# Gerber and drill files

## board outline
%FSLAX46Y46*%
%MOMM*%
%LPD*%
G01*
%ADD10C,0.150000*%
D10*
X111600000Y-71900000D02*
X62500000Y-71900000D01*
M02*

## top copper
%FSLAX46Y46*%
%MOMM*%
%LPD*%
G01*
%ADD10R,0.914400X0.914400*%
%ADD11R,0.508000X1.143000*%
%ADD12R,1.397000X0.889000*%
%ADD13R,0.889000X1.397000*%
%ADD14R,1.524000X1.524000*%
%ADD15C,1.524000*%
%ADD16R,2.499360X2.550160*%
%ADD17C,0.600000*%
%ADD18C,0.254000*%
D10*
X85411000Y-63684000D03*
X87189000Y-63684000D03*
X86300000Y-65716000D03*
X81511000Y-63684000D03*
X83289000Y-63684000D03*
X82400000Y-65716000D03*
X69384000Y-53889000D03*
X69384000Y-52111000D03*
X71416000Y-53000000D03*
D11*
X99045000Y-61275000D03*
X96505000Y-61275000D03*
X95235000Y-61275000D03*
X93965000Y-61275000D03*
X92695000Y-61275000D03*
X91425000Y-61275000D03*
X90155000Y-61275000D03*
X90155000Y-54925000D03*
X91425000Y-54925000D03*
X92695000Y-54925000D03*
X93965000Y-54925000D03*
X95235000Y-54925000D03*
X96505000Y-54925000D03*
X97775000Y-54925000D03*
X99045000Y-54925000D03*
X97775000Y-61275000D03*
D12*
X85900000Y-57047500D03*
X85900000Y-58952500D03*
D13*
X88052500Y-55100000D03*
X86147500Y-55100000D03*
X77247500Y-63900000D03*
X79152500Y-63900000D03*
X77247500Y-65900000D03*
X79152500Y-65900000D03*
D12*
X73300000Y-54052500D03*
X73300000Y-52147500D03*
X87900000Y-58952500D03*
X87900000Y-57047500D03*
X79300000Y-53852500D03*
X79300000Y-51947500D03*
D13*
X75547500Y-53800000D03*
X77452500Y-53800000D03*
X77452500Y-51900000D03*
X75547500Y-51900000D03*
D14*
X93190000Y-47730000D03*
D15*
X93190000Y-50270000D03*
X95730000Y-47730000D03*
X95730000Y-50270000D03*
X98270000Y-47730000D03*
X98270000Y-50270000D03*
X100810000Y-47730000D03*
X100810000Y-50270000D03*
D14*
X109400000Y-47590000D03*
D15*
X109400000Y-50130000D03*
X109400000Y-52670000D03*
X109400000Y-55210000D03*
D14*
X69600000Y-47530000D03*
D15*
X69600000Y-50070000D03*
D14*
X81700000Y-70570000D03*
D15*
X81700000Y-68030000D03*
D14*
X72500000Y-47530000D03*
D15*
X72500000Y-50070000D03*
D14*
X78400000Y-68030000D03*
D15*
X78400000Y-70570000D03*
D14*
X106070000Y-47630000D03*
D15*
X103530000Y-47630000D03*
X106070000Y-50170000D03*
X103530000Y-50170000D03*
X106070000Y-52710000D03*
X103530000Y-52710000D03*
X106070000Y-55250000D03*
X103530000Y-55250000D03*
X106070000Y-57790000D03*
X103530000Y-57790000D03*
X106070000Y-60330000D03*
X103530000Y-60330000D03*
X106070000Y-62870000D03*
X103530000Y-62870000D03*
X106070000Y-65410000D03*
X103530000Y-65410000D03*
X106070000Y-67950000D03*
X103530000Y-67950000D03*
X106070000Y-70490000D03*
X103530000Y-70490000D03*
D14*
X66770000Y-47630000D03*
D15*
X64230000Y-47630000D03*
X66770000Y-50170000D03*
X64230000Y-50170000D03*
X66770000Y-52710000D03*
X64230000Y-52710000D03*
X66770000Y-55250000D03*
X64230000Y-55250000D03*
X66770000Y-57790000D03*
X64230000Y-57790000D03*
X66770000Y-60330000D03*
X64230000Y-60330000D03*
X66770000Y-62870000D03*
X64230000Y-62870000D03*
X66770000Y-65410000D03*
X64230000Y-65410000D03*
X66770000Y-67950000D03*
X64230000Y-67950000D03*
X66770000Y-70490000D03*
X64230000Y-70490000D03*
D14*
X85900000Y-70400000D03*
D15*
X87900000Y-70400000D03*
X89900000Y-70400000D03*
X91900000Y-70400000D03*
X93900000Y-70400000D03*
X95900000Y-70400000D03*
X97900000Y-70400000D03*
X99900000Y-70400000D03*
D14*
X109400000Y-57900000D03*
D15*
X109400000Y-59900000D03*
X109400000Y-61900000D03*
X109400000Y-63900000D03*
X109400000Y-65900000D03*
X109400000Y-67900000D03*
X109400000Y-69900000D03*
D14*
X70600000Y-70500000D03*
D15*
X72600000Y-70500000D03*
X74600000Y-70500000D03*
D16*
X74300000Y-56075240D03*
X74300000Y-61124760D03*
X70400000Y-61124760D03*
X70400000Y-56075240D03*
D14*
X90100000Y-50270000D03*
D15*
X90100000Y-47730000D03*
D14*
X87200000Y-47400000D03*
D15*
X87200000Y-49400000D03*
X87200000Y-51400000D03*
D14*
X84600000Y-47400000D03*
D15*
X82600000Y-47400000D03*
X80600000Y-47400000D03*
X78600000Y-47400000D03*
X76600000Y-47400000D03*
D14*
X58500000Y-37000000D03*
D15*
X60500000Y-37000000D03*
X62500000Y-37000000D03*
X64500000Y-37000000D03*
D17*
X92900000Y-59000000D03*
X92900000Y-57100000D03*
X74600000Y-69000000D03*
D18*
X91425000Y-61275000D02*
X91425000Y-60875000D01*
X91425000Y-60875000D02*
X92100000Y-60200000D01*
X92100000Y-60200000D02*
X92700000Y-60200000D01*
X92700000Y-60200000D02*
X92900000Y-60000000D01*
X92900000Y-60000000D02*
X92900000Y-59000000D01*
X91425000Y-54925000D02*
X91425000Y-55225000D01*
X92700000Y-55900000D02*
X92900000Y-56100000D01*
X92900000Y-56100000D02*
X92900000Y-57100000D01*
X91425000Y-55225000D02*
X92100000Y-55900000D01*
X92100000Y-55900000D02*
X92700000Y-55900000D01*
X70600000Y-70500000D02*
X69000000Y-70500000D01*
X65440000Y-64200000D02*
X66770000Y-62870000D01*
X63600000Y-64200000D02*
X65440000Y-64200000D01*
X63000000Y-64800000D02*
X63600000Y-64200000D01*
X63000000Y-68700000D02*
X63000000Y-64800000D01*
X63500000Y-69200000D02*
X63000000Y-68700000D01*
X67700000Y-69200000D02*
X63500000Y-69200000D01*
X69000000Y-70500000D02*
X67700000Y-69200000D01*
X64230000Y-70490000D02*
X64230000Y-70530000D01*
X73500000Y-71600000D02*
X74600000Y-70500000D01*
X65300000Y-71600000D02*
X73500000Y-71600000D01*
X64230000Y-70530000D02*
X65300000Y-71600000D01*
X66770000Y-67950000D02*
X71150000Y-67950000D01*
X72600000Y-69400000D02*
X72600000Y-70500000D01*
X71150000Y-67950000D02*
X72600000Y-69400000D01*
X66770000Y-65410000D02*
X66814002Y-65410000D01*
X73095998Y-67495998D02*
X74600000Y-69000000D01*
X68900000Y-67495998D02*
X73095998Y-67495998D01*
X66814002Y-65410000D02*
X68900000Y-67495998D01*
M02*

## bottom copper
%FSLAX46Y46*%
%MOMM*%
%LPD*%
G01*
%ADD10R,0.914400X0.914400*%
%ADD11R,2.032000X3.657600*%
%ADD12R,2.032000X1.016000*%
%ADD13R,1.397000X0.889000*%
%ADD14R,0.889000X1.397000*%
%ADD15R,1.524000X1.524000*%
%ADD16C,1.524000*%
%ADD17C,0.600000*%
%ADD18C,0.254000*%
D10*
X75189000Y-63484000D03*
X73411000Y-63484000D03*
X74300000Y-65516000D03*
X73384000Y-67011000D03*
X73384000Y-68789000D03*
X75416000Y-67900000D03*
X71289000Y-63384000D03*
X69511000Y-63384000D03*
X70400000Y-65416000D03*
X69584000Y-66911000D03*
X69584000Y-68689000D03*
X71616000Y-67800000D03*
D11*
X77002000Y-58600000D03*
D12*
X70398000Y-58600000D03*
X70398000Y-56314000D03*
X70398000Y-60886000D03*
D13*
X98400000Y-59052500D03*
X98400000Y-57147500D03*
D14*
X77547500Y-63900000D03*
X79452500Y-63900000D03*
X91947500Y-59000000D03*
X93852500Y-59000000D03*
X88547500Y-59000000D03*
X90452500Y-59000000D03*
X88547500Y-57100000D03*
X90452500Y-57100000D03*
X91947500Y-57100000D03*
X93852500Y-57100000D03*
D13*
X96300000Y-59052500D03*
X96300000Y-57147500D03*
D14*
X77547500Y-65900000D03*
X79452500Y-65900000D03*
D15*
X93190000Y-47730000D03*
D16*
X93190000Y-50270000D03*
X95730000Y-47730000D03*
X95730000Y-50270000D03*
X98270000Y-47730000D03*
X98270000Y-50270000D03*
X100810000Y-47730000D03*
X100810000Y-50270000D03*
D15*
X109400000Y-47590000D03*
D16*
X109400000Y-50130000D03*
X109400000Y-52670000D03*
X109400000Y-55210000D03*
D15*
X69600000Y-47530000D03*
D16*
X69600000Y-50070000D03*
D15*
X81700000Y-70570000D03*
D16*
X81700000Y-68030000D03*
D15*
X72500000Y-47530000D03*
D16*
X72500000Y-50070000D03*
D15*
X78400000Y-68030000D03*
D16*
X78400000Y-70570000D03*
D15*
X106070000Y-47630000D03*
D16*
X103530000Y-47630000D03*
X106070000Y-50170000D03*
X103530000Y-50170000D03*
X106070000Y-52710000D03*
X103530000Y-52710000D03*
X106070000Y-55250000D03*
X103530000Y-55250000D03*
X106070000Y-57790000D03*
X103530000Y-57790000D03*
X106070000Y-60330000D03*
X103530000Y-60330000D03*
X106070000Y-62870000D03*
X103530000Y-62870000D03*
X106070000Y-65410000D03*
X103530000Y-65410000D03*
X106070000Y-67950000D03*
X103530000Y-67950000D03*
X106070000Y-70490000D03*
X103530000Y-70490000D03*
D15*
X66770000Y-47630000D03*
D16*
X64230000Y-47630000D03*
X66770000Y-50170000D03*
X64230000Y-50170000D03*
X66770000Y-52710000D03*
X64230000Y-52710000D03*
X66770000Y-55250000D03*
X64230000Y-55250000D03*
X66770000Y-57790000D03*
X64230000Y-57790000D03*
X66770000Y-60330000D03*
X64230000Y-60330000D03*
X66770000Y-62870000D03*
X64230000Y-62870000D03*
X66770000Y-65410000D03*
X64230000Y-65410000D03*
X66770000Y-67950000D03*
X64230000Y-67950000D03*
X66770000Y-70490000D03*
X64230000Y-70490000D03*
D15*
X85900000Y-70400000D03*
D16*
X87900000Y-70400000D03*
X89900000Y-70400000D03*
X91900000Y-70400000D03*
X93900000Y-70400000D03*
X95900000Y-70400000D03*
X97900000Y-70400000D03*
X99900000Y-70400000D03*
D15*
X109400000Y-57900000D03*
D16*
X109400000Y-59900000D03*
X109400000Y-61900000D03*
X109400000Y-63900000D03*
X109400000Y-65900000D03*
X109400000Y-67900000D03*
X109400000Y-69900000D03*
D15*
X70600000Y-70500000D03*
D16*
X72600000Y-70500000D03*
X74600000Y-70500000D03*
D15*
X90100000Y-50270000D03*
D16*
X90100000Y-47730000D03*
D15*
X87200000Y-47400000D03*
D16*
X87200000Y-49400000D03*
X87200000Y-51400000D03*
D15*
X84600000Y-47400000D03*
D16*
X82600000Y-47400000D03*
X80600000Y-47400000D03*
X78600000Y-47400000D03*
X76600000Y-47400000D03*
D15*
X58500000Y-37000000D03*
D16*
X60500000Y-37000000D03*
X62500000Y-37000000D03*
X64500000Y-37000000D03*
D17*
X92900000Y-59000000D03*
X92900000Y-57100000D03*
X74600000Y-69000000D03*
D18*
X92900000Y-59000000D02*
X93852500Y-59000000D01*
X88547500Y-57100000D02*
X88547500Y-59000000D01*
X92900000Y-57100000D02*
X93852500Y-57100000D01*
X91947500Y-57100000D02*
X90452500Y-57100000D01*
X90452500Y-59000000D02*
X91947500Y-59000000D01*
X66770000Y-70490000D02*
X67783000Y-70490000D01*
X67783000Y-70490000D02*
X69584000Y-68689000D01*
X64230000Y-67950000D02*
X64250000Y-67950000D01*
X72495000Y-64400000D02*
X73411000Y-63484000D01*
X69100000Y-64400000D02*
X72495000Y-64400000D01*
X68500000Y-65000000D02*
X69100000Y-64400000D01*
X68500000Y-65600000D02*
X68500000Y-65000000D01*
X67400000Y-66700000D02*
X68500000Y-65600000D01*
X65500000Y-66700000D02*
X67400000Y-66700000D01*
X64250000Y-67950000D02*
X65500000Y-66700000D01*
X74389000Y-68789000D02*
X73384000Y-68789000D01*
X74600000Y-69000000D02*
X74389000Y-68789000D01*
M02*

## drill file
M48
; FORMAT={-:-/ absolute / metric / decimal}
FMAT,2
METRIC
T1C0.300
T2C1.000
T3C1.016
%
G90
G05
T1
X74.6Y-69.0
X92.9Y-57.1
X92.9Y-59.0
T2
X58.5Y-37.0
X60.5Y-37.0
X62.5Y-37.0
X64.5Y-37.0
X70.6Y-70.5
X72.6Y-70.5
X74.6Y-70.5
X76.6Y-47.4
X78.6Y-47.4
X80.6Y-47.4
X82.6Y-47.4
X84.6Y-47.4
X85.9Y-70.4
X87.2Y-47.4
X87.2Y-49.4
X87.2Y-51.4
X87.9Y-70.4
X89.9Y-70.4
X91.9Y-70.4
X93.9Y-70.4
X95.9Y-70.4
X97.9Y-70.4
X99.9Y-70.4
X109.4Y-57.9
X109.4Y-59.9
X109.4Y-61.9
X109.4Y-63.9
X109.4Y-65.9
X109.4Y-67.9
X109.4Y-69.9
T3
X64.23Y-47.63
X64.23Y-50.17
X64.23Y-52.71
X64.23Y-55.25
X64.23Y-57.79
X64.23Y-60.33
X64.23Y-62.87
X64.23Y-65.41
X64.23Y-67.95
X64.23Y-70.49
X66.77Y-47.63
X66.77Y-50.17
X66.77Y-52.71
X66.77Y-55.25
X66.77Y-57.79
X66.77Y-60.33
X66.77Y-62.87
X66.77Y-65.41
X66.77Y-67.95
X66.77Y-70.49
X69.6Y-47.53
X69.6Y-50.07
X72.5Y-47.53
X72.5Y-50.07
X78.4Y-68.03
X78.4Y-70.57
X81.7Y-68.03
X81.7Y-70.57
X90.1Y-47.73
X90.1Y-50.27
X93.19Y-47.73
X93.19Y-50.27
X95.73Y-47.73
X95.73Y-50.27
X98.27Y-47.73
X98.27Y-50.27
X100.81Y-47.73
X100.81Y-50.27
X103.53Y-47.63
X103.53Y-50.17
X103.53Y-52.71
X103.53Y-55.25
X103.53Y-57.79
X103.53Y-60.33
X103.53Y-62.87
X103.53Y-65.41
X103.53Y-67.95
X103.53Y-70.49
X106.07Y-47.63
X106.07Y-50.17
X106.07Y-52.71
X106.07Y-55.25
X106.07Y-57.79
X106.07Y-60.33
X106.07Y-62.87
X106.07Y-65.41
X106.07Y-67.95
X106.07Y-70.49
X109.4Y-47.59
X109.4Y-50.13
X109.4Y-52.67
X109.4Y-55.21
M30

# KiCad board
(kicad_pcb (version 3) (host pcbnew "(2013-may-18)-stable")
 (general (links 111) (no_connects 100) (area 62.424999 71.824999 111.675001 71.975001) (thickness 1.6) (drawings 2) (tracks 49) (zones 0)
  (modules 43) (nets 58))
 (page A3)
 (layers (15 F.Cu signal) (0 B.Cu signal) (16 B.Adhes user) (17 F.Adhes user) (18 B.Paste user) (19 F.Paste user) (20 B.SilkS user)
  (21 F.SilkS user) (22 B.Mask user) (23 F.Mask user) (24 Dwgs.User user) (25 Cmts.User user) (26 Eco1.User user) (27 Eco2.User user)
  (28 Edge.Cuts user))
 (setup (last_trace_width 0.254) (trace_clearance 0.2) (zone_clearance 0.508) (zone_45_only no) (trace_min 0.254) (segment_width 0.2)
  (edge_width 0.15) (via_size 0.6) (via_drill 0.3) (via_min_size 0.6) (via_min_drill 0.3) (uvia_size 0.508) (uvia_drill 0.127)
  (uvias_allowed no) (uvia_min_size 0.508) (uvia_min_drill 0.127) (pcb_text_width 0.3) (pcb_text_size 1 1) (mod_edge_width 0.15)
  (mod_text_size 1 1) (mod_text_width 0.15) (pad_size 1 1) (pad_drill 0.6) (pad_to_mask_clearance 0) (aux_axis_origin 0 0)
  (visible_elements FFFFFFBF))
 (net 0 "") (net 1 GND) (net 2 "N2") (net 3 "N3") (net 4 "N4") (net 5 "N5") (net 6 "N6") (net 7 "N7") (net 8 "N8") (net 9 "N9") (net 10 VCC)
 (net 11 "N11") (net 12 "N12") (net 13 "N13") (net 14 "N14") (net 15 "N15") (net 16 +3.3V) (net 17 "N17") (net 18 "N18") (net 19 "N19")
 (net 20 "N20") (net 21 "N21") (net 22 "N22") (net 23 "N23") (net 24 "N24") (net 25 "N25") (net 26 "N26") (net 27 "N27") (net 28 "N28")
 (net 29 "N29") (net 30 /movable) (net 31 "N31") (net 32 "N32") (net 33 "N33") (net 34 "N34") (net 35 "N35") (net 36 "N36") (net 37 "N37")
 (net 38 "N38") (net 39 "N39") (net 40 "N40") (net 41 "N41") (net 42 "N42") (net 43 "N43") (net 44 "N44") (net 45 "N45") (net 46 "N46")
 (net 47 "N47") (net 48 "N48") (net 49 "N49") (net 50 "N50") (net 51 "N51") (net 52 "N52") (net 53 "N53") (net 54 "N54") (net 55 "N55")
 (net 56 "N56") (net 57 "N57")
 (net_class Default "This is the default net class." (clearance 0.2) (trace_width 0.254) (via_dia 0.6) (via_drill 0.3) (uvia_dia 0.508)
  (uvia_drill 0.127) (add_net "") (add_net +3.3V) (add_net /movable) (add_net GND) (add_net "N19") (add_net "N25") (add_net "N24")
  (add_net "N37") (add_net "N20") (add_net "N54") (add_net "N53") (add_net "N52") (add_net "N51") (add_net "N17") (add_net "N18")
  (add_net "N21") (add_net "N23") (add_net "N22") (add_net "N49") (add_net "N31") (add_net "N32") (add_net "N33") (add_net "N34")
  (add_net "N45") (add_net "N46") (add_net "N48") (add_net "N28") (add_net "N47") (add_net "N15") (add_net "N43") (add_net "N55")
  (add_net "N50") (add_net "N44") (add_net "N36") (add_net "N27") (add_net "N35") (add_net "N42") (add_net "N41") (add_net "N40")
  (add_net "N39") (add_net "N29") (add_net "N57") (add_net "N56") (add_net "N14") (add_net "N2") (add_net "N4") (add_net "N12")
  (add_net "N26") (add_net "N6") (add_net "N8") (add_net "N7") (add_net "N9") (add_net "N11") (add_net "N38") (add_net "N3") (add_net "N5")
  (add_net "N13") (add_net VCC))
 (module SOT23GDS (layer B.Cu) (at 74.3 64.5 180)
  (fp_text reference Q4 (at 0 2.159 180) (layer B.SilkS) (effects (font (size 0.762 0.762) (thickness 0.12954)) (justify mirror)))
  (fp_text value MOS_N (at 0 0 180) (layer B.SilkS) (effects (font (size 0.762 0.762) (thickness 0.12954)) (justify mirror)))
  (pad S smd rect (at -0.889 1.016 180) (size 0.9144 0.9144) (layers B.Cu B.Paste B.Mask) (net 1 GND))
  (pad G smd rect (at 0.889 1.016 180) (size 0.9144 0.9144) (layers B.Cu B.Paste B.Mask) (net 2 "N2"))
  (pad D smd rect (at 0 -1.016 180) (size 0.9144 0.9144) (layers B.Cu B.Paste B.Mask) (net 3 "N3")))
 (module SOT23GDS (layer B.Cu) (at 74.4 67.9 270)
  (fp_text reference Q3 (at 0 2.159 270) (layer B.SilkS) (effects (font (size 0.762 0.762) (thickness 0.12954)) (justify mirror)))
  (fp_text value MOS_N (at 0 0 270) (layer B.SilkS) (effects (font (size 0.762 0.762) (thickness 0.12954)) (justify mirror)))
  (pad S smd rect (at -0.889 1.016 270) (size 0.9144 0.9144) (layers B.Cu B.Paste B.Mask) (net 1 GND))
  (pad G smd rect (at 0.889 1.016 270) (size 0.9144 0.9144) (layers B.Cu B.Paste B.Mask) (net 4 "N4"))
  (pad D smd rect (at 0 -1.016 270) (size 0.9144 0.9144) (layers B.Cu B.Paste B.Mask) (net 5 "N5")))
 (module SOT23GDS (layer F.Cu) (at 86.3 64.7)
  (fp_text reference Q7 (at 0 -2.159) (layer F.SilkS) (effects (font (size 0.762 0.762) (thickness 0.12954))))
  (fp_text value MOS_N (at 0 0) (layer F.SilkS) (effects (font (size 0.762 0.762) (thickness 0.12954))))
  (pad S smd rect (at -0.889 -1.016) (size 0.9144 0.9144) (layers F.Cu F.Paste F.Mask) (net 1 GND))
  (pad G smd rect (at 0.889 -1.016) (size 0.9144 0.9144) (layers F.Cu F.Paste F.Mask) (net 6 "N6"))
  (pad D smd rect (at 0 1.016) (size 0.9144 0.9144) (layers F.Cu F.Paste F.Mask) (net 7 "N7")))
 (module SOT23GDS (layer F.Cu) (at 82.4 64.7)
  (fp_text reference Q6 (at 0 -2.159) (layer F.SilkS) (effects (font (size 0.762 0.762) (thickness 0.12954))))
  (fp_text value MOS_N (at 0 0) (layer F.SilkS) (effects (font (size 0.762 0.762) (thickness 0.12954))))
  (pad S smd rect (at -0.889 -1.016) (size 0.9144 0.9144) (layers F.Cu F.Paste F.Mask) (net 1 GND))
  (pad G smd rect (at 0.889 -1.016) (size 0.9144 0.9144) (layers F.Cu F.Paste F.Mask) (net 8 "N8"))
  (pad D smd rect (at 0 1.016) (size 0.9144 0.9144) (layers F.Cu F.Paste F.Mask) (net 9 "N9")))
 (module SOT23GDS (layer F.Cu) (at 70.4 53 90)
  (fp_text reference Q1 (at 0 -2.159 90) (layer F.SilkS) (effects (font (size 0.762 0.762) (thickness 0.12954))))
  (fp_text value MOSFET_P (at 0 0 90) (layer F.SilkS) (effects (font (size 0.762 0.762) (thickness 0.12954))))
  (pad S smd rect (at -0.889 -1.016 90) (size 0.9144 0.9144) (layers F.Cu F.Paste F.Mask) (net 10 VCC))
  (pad G smd rect (at 0.889 -1.016 90) (size 0.9144 0.9144) (layers F.Cu F.Paste F.Mask) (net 1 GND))
  (pad D smd rect (at 0 1.016 90) (size 0.9144 0.9144) (layers F.Cu F.Paste F.Mask) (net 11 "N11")))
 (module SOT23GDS (layer B.Cu) (at 70.4 64.4 180)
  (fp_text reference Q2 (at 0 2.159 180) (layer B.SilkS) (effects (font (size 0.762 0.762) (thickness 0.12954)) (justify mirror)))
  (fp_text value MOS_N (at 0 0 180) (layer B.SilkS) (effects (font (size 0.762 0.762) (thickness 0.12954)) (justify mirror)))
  (pad S smd rect (at -0.889 1.016 180) (size 0.9144 0.9144) (layers B.Cu B.Paste B.Mask) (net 1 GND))
  (pad G smd rect (at 0.889 1.016 180) (size 0.9144 0.9144) (layers B.Cu B.Paste B.Mask) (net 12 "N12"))
  (pad D smd rect (at 0 -1.016 180) (size 0.9144 0.9144) (layers B.Cu B.Paste B.Mask) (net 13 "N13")))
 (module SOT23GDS (layer B.Cu) (at 70.6 67.8 270)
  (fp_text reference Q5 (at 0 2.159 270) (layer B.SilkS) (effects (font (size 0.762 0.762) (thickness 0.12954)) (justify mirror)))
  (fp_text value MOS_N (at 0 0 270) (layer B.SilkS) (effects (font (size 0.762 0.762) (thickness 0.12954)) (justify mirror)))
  (pad S smd rect (at -0.889 1.016 270) (size 0.9144 0.9144) (layers B.Cu B.Paste B.Mask) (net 1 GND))
  (pad G smd rect (at 0.889 1.016 270) (size 0.9144 0.9144) (layers B.Cu B.Paste B.Mask) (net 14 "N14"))
  (pad D smd rect (at 0 -1.016 270) (size 0.9144 0.9144) (layers B.Cu B.Paste B.Mask) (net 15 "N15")))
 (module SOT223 (layer B.Cu) (at 73.7 58.6 90)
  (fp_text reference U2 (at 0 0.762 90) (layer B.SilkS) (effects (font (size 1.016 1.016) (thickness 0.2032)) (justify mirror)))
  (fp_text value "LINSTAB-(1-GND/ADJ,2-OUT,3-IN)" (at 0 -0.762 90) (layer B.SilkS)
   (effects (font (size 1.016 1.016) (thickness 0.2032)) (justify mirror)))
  (pad 4 smd rect (at 0 3.302 90) (size 3.6576 2.032) (layers B.Cu B.Paste B.Mask))
  (pad 2 smd rect (at 0 -3.302 90) (size 1.016 2.032) (layers B.Cu B.Paste B.Mask) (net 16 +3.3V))
  (pad 3 smd rect (at 2.286 -3.302 90) (size 1.016 2.032) (layers B.Cu B.Paste B.Mask) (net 10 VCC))
  (pad 1 smd rect (at -2.286 -3.302 90) (size 1.016 2.032) (layers B.Cu B.Paste B.Mask) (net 1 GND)))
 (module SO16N (layer F.Cu) (at 94.6 58.1 180)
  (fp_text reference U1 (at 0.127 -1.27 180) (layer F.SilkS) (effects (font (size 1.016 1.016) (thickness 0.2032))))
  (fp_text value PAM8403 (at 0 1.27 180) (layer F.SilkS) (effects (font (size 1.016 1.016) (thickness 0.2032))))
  (pad 16 smd rect (at -4.445 -3.175 180) (size 0.508 1.143) (layers F.Cu F.Paste F.Mask) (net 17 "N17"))
  (pad 14 smd rect (at -1.905 -3.175 180) (size 0.508 1.143) (layers F.Cu F.Paste F.Mask) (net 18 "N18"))
  (pad 13 smd rect (at -0.635 -3.175 180) (size 0.508 1.143) (layers F.Cu F.Paste F.Mask) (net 10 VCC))
  (pad 12 smd rect (at 0.635 -3.175 180) (size 0.508 1.143) (layers F.Cu F.Paste F.Mask) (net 10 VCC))
  (pad 11 smd rect (at 1.905 -3.175 180) (size 0.508 1.143) (layers F.Cu F.Paste F.Mask) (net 1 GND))
  (pad 10 smd rect (at 3.175 -3.175 180) (size 0.508 1.143) (layers F.Cu F.Paste F.Mask) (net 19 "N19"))
  (pad 9 smd rect (at 4.445 -3.175 180) (size 0.508 1.143) (layers F.Cu F.Paste F.Mask) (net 1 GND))
  (pad 8 smd rect (at 4.445 3.175 180) (size 0.508 1.143) (layers F.Cu F.Paste F.Mask) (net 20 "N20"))
  (pad 7 smd rect (at 3.175 3.175 180) (size 0.508 1.143) (layers F.Cu F.Paste F.Mask) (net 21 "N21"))
  (pad 6 smd rect (at 1.905 3.175 180) (size 0.508 1.143) (layers F.Cu F.Paste F.Mask) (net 10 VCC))
  (pad 5 smd rect (at 0.635 3.175 180) (size 0.508 1.143) (layers F.Cu F.Paste F.Mask) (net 10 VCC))
  (pad 4 smd rect (at -0.635 3.175 180) (size 0.508 1.143) (layers F.Cu F.Paste F.Mask) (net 10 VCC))
  (pad 3 smd rect (at -1.905 3.175 180) (size 0.508 1.143) (layers F.Cu F.Paste F.Mask) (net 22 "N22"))
  (pad 2 smd rect (at -3.175 3.175 180) (size 0.508 1.143) (layers F.Cu F.Paste F.Mask) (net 1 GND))
  (pad 1 smd rect (at -4.445 3.175 180) (size 0.508 1.143) (layers F.Cu F.Paste F.Mask) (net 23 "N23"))
  (pad 15 smd rect (at -3.175 -3.175 180) (size 0.508 1.143) (layers F.Cu F.Paste F.Mask) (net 1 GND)))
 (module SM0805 (layer B.Cu) (at 98.4 58.1 90)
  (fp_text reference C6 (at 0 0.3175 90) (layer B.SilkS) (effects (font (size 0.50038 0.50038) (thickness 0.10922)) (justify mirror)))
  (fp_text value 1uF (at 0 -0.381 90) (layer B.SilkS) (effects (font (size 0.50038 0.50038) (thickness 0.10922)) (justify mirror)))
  (pad 1 smd rect (at -0.9525 0 90) (size 0.889 1.397) (layers B.Cu B.Paste B.Mask) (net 10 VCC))
  (pad 2 smd rect (at 0.9525 0 90) (size 0.889 1.397) (layers B.Cu B.Paste B.Mask) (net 1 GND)))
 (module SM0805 (layer F.Cu) (at 85.9 58 270)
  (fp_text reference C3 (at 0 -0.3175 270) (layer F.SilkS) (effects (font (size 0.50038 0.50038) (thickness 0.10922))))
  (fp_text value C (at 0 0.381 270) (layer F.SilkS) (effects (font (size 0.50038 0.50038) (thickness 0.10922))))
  (pad 1 smd rect (at -0.9525 0 270) (size 0.889 1.397) (layers F.Cu F.Paste F.Mask) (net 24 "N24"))
  (pad 2 smd rect (at 0.9525 0 270) (size 0.889 1.397) (layers F.Cu F.Paste F.Mask) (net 1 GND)))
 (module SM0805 (layer F.Cu) (at 87.1 55.1 180)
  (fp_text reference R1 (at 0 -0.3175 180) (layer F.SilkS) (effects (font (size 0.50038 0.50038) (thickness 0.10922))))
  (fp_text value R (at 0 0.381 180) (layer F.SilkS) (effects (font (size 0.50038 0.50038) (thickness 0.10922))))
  (pad 1 smd rect (at -0.9525 0 180) (size 0.889 1.397) (layers F.Cu F.Paste F.Mask) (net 24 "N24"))
  (pad 2 smd rect (at 0.9525 0 180) (size 0.889 1.397) (layers F.Cu F.Paste F.Mask) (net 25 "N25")))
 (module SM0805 (layer F.Cu) (at 78.2 63.9)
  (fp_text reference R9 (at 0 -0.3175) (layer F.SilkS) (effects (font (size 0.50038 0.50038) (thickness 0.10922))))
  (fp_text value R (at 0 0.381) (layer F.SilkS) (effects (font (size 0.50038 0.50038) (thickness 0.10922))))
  (pad 1 smd rect (at -0.9525 0) (size 0.889 1.397) (layers F.Cu F.Paste F.Mask) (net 15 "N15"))
  (pad 2 smd rect (at 0.9525 0) (size 0.889 1.397) (layers F.Cu F.Paste F.Mask) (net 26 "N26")))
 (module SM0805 (layer B.Cu) (at 78.5 63.9)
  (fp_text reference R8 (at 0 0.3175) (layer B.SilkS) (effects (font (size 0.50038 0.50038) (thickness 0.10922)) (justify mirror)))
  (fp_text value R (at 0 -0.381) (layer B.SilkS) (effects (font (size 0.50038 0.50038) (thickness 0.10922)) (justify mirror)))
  (pad 1 smd rect (at -0.9525 0) (size 0.889 1.397) (layers B.Cu B.Paste B.Mask) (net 3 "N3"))
  (pad 2 smd rect (at 0.9525 0) (size 0.889 1.397) (layers B.Cu B.Paste B.Mask) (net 26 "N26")))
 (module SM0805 (layer F.Cu) (at 78.2 65.9)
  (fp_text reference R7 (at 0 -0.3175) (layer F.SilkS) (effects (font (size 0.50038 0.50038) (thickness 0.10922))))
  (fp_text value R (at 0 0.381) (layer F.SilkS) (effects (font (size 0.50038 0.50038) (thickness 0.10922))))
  (pad 1 smd rect (at -0.9525 0) (size 0.889 1.397) (layers F.Cu F.Paste F.Mask) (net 5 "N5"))
  (pad 2 smd rect (at 0.9525 0) (size 0.889 1.397) (layers F.Cu F.Paste F.Mask) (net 26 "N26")))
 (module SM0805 (layer B.Cu) (at 92.9 59)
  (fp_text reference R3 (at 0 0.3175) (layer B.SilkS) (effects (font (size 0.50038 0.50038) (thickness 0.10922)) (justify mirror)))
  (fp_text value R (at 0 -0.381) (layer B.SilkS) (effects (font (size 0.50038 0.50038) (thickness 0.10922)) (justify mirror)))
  (pad 1 smd rect (at -0.9525 0) (size 0.889 1.397) (layers B.Cu B.Paste B.Mask) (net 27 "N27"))
  (pad 2 smd rect (at 0.9525 0) (size 0.889 1.397) (layers B.Cu B.Paste B.Mask) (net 19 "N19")))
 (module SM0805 (layer B.Cu) (at 89.5 59)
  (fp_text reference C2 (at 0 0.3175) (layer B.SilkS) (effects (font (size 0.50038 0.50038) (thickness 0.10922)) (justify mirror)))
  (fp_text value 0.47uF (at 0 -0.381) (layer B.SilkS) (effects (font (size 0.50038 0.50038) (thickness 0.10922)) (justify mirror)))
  (pad 1 smd rect (at -0.9525 0) (size 0.889 1.397) (layers B.Cu B.Paste B.Mask) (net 24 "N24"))
  (pad 2 smd rect (at 0.9525 0) (size 0.889 1.397) (layers B.Cu B.Paste B.Mask) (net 27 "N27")))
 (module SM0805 (layer B.Cu) (at 89.5 57.1)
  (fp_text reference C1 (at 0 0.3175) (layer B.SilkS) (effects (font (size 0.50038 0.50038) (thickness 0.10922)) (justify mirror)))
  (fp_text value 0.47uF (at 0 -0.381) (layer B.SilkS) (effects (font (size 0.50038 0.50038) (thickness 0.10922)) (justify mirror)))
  (pad 1 smd rect (at -0.9525 0) (size 0.889 1.397) (layers B.Cu B.Paste B.Mask) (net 24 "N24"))
  (pad 2 smd rect (at 0.9525 0) (size 0.889 1.397) (layers B.Cu B.Paste B.Mask) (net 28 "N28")))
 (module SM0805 (layer B.Cu) (at 92.9 57.1)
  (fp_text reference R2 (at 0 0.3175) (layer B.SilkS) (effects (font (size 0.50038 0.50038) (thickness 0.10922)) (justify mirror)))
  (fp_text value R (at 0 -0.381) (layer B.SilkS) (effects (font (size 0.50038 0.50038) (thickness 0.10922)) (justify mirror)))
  (pad 1 smd rect (at -0.9525 0) (size 0.889 1.397) (layers B.Cu B.Paste B.Mask) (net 28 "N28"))
  (pad 2 smd rect (at 0.9525 0) (size 0.889 1.397) (layers B.Cu B.Paste B.Mask) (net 21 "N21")))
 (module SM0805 (layer F.Cu) (at 73.3 53.1 90)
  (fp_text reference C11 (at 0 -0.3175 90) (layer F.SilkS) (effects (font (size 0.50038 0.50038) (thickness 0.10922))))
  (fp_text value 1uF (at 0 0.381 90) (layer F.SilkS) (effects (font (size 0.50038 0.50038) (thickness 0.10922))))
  (pad 1 smd rect (at -0.9525 0 90) (size 0.889 1.397) (layers F.Cu F.Paste F.Mask) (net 10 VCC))
  (pad 2 smd rect (at 0.9525 0 90) (size 0.889 1.397) (layers F.Cu F.Paste F.Mask) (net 1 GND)))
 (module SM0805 (layer B.Cu) (at 96.3 58.1 90)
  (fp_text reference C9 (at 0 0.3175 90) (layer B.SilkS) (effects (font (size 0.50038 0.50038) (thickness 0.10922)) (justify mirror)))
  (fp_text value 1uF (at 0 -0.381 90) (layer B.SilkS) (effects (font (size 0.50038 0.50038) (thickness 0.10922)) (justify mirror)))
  (pad 1 smd rect (at -0.9525 0 90) (size 0.889 1.397) (layers B.Cu B.Paste B.Mask) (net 10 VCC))
  (pad 2 smd rect (at 0.9525 0 90) (size 0.889 1.397) (layers B.Cu B.Paste B.Mask) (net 1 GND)))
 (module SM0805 (layer B.Cu) (at 78.5 65.9)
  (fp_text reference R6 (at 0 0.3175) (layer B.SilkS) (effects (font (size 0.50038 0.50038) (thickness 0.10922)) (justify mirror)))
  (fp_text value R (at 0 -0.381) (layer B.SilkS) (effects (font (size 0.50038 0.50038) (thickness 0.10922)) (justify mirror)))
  (pad 1 smd rect (at -0.9525 0) (size 0.889 1.397) (layers B.Cu B.Paste B.Mask) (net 13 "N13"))
  (pad 2 smd rect (at 0.9525 0) (size 0.889 1.397) (layers B.Cu B.Paste B.Mask) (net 26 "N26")))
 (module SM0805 (layer F.Cu) (at 87.9 58 90)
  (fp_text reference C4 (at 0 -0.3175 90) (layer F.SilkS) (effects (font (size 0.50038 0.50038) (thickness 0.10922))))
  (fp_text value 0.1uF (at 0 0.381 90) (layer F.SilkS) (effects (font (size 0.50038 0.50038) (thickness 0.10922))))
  (pad 1 smd rect (at -0.9525 0 90) (size 0.889 1.397) (layers F.Cu F.Paste F.Mask) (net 1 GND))
  (pad 2 smd rect (at 0.9525 0 90) (size 0.889 1.397) (layers F.Cu F.Paste F.Mask) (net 20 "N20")))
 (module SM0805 (layer F.Cu) (at 79.3 52.9 90)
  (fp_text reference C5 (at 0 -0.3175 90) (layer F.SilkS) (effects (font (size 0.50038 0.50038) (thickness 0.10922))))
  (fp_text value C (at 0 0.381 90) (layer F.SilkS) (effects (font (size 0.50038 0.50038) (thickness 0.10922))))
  (pad 1 smd rect (at -0.9525 0 90) (size 0.889 1.397) (layers F.Cu F.Paste F.Mask) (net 10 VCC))
  (pad 2 smd rect (at 0.9525 0 90) (size 0.889 1.397) (layers F.Cu F.Paste F.Mask) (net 1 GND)))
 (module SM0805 (layer F.Cu) (at 76.5 53.8)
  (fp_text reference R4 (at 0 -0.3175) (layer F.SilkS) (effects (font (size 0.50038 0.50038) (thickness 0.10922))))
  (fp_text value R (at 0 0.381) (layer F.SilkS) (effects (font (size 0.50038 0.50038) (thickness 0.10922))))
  (pad 1 smd rect (at -0.9525 0) (size 0.889 1.397) (layers F.Cu F.Paste F.Mask) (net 10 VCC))
  (pad 2 smd rect (at 0.9525 0) (size 0.889 1.397) (layers F.Cu F.Paste F.Mask) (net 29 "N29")))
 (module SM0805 (layer F.Cu) (at 76.5 51.9 180)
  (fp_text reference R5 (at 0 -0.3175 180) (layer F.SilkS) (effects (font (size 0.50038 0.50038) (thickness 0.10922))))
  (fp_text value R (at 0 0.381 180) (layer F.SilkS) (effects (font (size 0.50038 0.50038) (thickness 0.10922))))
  (pad 1 smd rect (at -0.9525 0 180) (size 0.889 1.397) (layers F.Cu F.Paste F.Mask) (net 29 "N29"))
  (pad 2 smd rect (at 0.9525 0 180) (size 0.889 1.397) (layers F.Cu F.Paste F.Mask) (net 1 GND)))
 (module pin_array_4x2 (layer B.Cu) (at 97 49)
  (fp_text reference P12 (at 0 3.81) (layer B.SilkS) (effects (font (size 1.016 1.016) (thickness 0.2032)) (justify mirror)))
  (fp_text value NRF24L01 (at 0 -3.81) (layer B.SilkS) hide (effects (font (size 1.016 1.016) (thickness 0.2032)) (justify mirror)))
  (pad 1 thru_hole rect (at -3.81 -1.27) (size 1.524 1.524) (drill 1.016) (layers *.Cu *.Mask B.SilkS) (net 1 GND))
  (pad 2 thru_hole circle (at -3.81 1.27) (size 1.524 1.524) (drill 1.016) (layers *.Cu *.Mask B.SilkS) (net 16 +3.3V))
  (pad 3 thru_hole circle (at -1.27 -1.27) (size 1.524 1.524) (drill 1.016) (layers *.Cu *.Mask B.SilkS) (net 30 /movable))
  (pad 4 thru_hole circle (at -1.27 1.27) (size 1.524 1.524) (drill 1.016) (layers *.Cu *.Mask B.SilkS) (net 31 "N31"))
  (pad 5 thru_hole circle (at 1.27 -1.27) (size 1.524 1.524) (drill 1.016) (layers *.Cu *.Mask B.SilkS) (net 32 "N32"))
  (pad 6 thru_hole circle (at 1.27 1.27) (size 1.524 1.524) (drill 1.016) (layers *.Cu *.Mask B.SilkS) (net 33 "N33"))
  (pad 7 thru_hole circle (at 3.81 -1.27) (size 1.524 1.524) (drill 1.016) (layers *.Cu *.Mask B.SilkS) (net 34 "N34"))
  (pad 8 thru_hole circle (at 3.81 1.27) (size 1.524 1.524) (drill 1.016) (layers *.Cu *.Mask B.SilkS) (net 30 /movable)))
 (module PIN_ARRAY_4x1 (layer B.Cu) (at 109.4 51.4 270)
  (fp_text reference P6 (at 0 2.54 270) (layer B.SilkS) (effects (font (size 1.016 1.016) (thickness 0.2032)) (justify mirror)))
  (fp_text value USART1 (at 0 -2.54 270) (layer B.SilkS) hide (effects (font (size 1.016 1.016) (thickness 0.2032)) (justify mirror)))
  (pad 1 thru_hole rect (at -3.81 0 270) (size 1.524 1.524) (drill 1.016) (layers *.Cu *.Mask B.SilkS) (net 1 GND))
  (pad 2 thru_hole circle (at -1.27 0 270) (size 1.524 1.524) (drill 1.016) (layers *.Cu *.Mask B.SilkS))
  (pad 3 thru_hole circle (at 1.27 0 270) (size 1.524 1.524) (drill 1.016) (layers *.Cu *.Mask B.SilkS) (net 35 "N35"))
  (pad 4 thru_hole circle (at 3.81 0 270) (size 1.524 1.524) (drill 1.016) (layers *.Cu *.Mask B.SilkS) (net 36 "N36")))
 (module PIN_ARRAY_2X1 (layer B.Cu) (at 69.6 48.8 270)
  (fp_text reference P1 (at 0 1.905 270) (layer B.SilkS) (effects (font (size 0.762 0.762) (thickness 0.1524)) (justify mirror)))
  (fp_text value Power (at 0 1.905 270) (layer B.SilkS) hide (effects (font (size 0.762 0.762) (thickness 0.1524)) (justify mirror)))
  (pad 1 thru_hole rect (at -1.27 0 270) (size 1.524 1.524) (drill 1.016) (layers *.Cu *.Mask B.SilkS) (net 1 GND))
  (pad 2 thru_hole circle (at 1.27 0 270) (size 1.524 1.524) (drill 1.016) (layers *.Cu *.Mask B.SilkS) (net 11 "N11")))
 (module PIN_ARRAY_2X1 (layer B.Cu) (at 81.7 69.3 90)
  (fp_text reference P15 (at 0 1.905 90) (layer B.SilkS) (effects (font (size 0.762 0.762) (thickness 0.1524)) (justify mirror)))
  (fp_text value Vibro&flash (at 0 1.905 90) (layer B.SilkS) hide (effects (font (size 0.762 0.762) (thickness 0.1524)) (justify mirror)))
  (pad 1 thru_hole rect (at -1.27 0 90) (size 1.524 1.524) (drill 1.016) (layers *.Cu *.Mask B.SilkS) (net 7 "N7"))
  (pad 2 thru_hole circle (at 1.27 0 90) (size 1.524 1.524) (drill 1.016) (layers *.Cu *.Mask B.SilkS) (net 9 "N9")))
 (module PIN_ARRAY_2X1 (layer B.Cu) (at 72.5 48.8 270)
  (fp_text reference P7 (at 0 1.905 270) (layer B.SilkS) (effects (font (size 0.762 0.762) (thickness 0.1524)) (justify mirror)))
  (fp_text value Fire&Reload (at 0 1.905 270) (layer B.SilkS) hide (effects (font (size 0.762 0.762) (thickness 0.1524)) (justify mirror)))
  (pad 1 thru_hole rect (at -1.27 0 270) (size 1.524 1.524) (drill 1.016) (layers *.Cu *.Mask B.SilkS) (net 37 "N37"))
  (pad 2 thru_hole circle (at 1.27 0 270) (size 1.524 1.524) (drill 1.016) (layers *.Cu *.Mask B.SilkS) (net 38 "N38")))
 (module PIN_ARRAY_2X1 (layer B.Cu) (at 78.4 69.3 270)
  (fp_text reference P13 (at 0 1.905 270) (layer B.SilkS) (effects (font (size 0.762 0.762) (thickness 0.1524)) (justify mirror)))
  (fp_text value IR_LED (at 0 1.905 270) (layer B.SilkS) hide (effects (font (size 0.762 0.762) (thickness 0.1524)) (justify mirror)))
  (pad 1 thru_hole rect (at -1.27 0 270) (size 1.524 1.524) (drill 1.016) (layers *.Cu *.Mask B.SilkS) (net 26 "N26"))
  (pad 2 thru_hole circle (at 1.27 0 270) (size 1.524 1.524) (drill 1.016) (layers *.Cu *.Mask B.SilkS) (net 10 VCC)))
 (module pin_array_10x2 (layer B.Cu) (at 104.8 59.1 270)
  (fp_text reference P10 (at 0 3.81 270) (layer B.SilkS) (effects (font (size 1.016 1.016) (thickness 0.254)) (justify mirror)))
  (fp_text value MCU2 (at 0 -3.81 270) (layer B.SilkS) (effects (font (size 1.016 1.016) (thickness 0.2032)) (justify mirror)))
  (pad 1 thru_hole rect (at -11.47 -1.27 270) (size 1.524 1.524) (drill 1.016) (layers *.Cu *.Mask B.SilkS) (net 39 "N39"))
  (pad 2 thru_hole circle (at -11.47 1.27 270) (size 1.524 1.524) (drill 1.016) (layers *.Cu *.Mask B.SilkS) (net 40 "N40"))
  (pad 3 thru_hole circle (at -8.93 -1.27 270) (size 1.524 1.524) (drill 1.016) (layers *.Cu *.Mask B.SilkS) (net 31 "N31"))
  (pad 4 thru_hole circle (at -8.93 1.27 270) (size 1.524 1.524) (drill 1.016) (layers *.Cu *.Mask B.SilkS) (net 32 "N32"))
  (pad 5 thru_hole circle (at -6.39 -1.27 270) (size 1.524 1.524) (drill 1.016) (layers *.Cu *.Mask B.SilkS) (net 34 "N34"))
  (pad 6 thru_hole circle (at -6.39 1.27 270) (size 1.524 1.524) (drill 1.016) (layers *.Cu *.Mask B.SilkS) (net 33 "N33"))
  (pad 7 thru_hole circle (at -3.85 -1.27 270) (size 1.524 1.524) (drill 1.016) (layers *.Cu *.Mask B.SilkS) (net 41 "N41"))
  (pad 8 thru_hole circle (at -3.85 1.27 270) (size 1.524 1.524) (drill 1.016) (layers *.Cu *.Mask B.SilkS) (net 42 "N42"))
  (pad 9 thru_hole circle (at -1.31 -1.27 270) (size 1.524 1.524) (drill 1.016) (layers *.Cu *.Mask B.SilkS) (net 35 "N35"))
  (pad 10 thru_hole circle (at -1.31 1.27 270) (size 1.524 1.524) (drill 1.016) (layers *.Cu *.Mask B.SilkS) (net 36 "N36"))
  (pad 11 thru_hole circle (at 1.23 -1.27 270) (size 1.524 1.524) (drill 1.016) (layers *.Cu *.Mask B.SilkS) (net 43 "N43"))
  (pad 12 thru_hole circle (at 1.23 1.27 270) (size 1.524 1.524) (drill 1.016) (layers *.Cu *.Mask B.SilkS) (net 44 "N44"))
  (pad 13 thru_hole circle (at 3.77 -1.27 270) (size 1.524 1.524) (drill 1.016) (layers *.Cu *.Mask B.SilkS) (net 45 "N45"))
  (pad 14 thru_hole circle (at 3.77 1.27 270) (size 1.524 1.524) (drill 1.016) (layers *.Cu *.Mask B.SilkS) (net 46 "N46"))
  (pad 15 thru_hole circle (at 6.31 -1.27 270) (size 1.524 1.524) (drill 1.016) (layers *.Cu *.Mask B.SilkS) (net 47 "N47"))
  (pad 16 thru_hole circle (at 6.31 1.27 270) (size 1.524 1.524) (drill 1.016) (layers *.Cu *.Mask B.SilkS) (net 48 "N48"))
  (pad 17 thru_hole circle (at 8.85 -1.27 270) (size 1.524 1.524) (drill 1.016) (layers *.Cu *.Mask B.SilkS) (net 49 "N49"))
  (pad 18 thru_hole circle (at 8.85 1.27 270) (size 1.524 1.524) (drill 1.016) (layers *.Cu *.Mask B.SilkS) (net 30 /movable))
  (pad 19 thru_hole circle (at 11.39 -1.27 270) (size 1.524 1.524) (drill 1.016) (layers *.Cu *.Mask B.SilkS) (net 30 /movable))
  (pad 20 thru_hole circle (at 11.39 1.27 270) (size 1.524 1.524) (drill 1.016) (layers *.Cu *.Mask B.SilkS) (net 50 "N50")))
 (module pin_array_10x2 (layer B.Cu) (at 65.5 59.1 270)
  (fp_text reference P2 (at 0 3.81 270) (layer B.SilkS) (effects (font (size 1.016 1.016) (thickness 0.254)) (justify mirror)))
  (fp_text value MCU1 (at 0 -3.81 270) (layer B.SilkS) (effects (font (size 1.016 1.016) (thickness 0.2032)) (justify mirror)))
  (pad 1 thru_hole rect (at -11.47 -1.27 270) (size 1.524 1.524) (drill 1.016) (layers *.Cu *.Mask B.SilkS) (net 1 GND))
  (pad 2 thru_hole circle (at -11.47 1.27 270) (size 1.524 1.524) (drill 1.016) (layers *.Cu *.Mask B.SilkS) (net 16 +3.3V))
  (pad 3 thru_hole circle (at -8.93 -1.27 270) (size 1.524 1.524) (drill 1.016) (layers *.Cu *.Mask B.SilkS))
  (pad 4 thru_hole circle (at -8.93 1.27 270) (size 1.524 1.524) (drill 1.016) (layers *.Cu *.Mask B.SilkS) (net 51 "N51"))
  (pad 5 thru_hole circle (at -6.39 -1.27 270) (size 1.524 1.524) (drill 1.016) (layers *.Cu *.Mask B.SilkS) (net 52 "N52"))
  (pad 6 thru_hole circle (at -6.39 1.27 270) (size 1.524 1.524) (drill 1.016) (layers *.Cu *.Mask B.SilkS) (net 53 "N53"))
  (pad 7 thru_hole circle (at -3.85 -1.27 270) (size 1.524 1.524) (drill 1.016) (layers *.Cu *.Mask B.SilkS) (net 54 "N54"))
  (pad 8 thru_hole circle (at -3.85 1.27 270) (size 1.524 1.524) (drill 1.016) (layers *.Cu *.Mask B.SilkS) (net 37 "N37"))
  (pad 9 thru_hole circle (at -1.31 -1.27 270) (size 1.524 1.524) (drill 1.016) (layers *.Cu *.Mask B.SilkS) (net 38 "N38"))
  (pad 10 thru_hole circle (at -1.31 1.27 270) (size 1.524 1.524) (drill 1.016) (layers *.Cu *.Mask B.SilkS) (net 8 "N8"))
  (pad 11 thru_hole circle (at 1.23 -1.27 270) (size 1.524 1.524) (drill 1.016) (layers *.Cu *.Mask B.SilkS) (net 6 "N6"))
  (pad 12 thru_hole circle (at 1.23 1.27 270) (size 1.524 1.524) (drill 1.016) (layers *.Cu *.Mask B.SilkS) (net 25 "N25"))
  (pad 13 thru_hole circle (at 3.77 -1.27 270) (size 1.524 1.524) (drill 1.016) (layers *.Cu *.Mask B.SilkS) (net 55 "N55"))
  (pad 14 thru_hole circle (at 3.77 1.27 270) (size 1.524 1.524) (drill 1.016) (layers *.Cu *.Mask B.SilkS) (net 12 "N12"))
  (pad 15 thru_hole circle (at 6.31 -1.27 270) (size 1.524 1.524) (drill 1.016) (layers *.Cu *.Mask B.SilkS) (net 4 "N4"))
  (pad 16 thru_hole circle (at 6.31 1.27 270) (size 1.524 1.524) (drill 1.016) (layers *.Cu *.Mask B.SilkS) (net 29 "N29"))
  (pad 17 thru_hole circle (at 8.85 -1.27 270) (size 1.524 1.524) (drill 1.016) (layers *.Cu *.Mask B.SilkS) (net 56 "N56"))
  (pad 18 thru_hole circle (at 8.85 1.27 270) (size 1.524 1.524) (drill 1.016) (layers *.Cu *.Mask B.SilkS) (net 2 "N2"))
  (pad 19 thru_hole circle (at 11.39 -1.27 270) (size 1.524 1.524) (drill 1.016) (layers *.Cu *.Mask B.SilkS) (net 14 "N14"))
  (pad 20 thru_hole circle (at 11.39 1.27 270) (size 1.524 1.524) (drill 1.016) (layers *.Cu *.Mask B.SilkS) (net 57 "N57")))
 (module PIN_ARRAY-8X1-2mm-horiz (layer B.Cu) (at 92.9 70.4)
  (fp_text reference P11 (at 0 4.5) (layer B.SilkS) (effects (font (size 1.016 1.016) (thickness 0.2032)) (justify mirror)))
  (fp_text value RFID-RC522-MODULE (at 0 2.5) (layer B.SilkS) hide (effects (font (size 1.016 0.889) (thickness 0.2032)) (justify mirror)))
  (pad 1 thru_hole rect (at -7 0) (size 1.524 1.524) (drill 1) (layers *.Cu *.Mask B.SilkS) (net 45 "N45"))
  (pad 2 thru_hole circle (at -5 0) (size 1.524 1.524) (drill 1) (layers *.Cu *.Mask B.SilkS) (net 46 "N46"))
  (pad 3 thru_hole circle (at -3 0) (size 1.524 1.524) (drill 1) (layers *.Cu *.Mask B.SilkS) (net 48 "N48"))
  (pad 4 thru_hole circle (at -1 0) (size 1.524 1.524) (drill 1) (layers *.Cu *.Mask B.SilkS) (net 47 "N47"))
  (pad 5 thru_hole circle (at 1 0) (size 1.524 1.524) (drill 1) (layers *.Cu *.Mask B.SilkS) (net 49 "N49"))
  (pad 6 thru_hole circle (at 3 0) (size 1.524 1.524) (drill 1) (layers *.Cu *.Mask B.SilkS) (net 1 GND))
  (pad 7 thru_hole circle (at 5 0) (size 1.524 1.524) (drill 1) (layers *.Cu *.Mask B.SilkS) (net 16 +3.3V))
  (pad 8 thru_hole circle (at 7 0) (size 1.524 1.524) (drill 1) (layers *.Cu *.Mask B.SilkS) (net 16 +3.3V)))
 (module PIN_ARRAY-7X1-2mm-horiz (layer F.Cu) (at 109.4 63.9 270)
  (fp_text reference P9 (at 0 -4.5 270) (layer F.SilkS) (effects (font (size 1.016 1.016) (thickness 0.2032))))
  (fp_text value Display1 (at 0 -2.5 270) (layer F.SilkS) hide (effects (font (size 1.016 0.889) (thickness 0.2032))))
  (pad 1 thru_hole rect (at -6 0 270) (size 1.524 1.524) (drill 1) (layers *.Cu *.Mask F.SilkS) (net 39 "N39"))
  (pad 2 thru_hole circle (at -4 0 270) (size 1.524 1.524) (drill 1) (layers *.Cu *.Mask F.SilkS) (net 40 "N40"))
  (pad 3 thru_hole circle (at -2 0 270) (size 1.524 1.524) (drill 1) (layers *.Cu *.Mask F.SilkS) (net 41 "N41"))
  (pad 4 thru_hole circle (at 0 0 270) (size 1.524 1.524) (drill 1) (layers *.Cu *.Mask F.SilkS) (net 42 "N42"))
  (pad 5 thru_hole circle (at 2 0 270) (size 1.524 1.524) (drill 1) (layers *.Cu *.Mask F.SilkS) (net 43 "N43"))
  (pad 6 thru_hole circle (at 4 0 270) (size 1.524 1.524) (drill 1) (layers *.Cu *.Mask F.SilkS) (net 44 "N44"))
  (pad 7 thru_hole circle (at 6 0 270) (size 1.524 1.524) (drill 1) (layers *.Cu *.Mask F.SilkS) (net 50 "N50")))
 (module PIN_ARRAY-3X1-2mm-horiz (layer B.Cu) (at 72.6 70.5)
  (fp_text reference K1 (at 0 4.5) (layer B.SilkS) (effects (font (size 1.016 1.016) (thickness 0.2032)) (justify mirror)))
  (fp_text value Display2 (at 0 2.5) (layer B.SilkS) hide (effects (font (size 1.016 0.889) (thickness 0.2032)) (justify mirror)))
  (pad 1 thru_hole rect (at -2 0) (size 1.524 1.524) (drill 1) (layers *.Cu *.Mask B.SilkS) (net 55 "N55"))
  (pad 2 thru_hole circle (at 0 0) (size 1.524 1.524) (drill 1) (layers *.Cu *.Mask B.SilkS) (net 56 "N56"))
  (pad 3 thru_hole circle (at 2 0) (size 1.524 1.524) (drill 1) (layers *.Cu *.Mask B.SilkS) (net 57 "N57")))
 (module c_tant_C (layer F.Cu) (at 74.3 58.6 90)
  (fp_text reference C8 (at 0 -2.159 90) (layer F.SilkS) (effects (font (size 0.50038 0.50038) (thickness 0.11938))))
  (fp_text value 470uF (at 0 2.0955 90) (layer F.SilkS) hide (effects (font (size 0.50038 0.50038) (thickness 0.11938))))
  (pad 1 smd rect (at 2.52476 0 90) (size 2.55016 2.49936) (layers F.Cu F.Paste F.Mask) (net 10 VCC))
  (pad 2 smd rect (at -2.52476 0 90) (size 2.55016 2.49936) (layers F.Cu F.Paste F.Mask) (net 1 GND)))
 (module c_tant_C (layer F.Cu) (at 70.4 58.6 270)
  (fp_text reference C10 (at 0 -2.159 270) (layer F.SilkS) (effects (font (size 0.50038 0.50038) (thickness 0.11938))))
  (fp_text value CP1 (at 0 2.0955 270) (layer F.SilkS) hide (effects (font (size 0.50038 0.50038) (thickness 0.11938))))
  (pad 1 smd rect (at 2.52476 0 270) (size 2.55016 2.49936) (layers F.Cu F.Paste F.Mask) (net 16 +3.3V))
  (pad 2 smd rect (at -2.52476 0 270) (size 2.55016 2.49936) (layers F.Cu F.Paste F.Mask) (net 1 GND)))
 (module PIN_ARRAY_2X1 (layer B.Cu) (at 90.1 49 90)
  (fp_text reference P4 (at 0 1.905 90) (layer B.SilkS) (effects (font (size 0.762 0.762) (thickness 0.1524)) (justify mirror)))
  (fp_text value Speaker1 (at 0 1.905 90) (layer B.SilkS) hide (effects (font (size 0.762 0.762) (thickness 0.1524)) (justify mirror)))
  (pad 1 thru_hole rect (at -1.27 0 90) (size 1.524 1.524) (drill 1.016) (layers *.Cu *.Mask B.SilkS) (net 22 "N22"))
  (pad 2 thru_hole circle (at 1.27 0 90) (size 1.524 1.524) (drill 1.016) (layers *.Cu *.Mask B.SilkS) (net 23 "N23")))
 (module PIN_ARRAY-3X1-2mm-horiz (layer B.Cu) (at 87.2 49.4 270)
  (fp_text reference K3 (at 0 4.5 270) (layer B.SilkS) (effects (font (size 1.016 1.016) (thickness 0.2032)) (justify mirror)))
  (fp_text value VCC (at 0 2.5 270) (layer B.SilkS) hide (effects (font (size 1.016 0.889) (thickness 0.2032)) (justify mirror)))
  (pad 1 thru_hole rect (at -2 0 270) (size 1.524 1.524) (drill 1) (layers *.Cu *.Mask B.SilkS) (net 10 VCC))
  (pad 2 thru_hole circle (at 0 0 270) (size 1.524 1.524) (drill 1) (layers *.Cu *.Mask B.SilkS) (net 10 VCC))
  (pad 3 thru_hole circle (at 2 0 270) (size 1.524 1.524) (drill 1) (layers *.Cu *.Mask B.SilkS) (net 10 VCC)))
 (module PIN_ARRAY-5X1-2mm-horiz (layer B.Cu) (at 80.6 47.4 180)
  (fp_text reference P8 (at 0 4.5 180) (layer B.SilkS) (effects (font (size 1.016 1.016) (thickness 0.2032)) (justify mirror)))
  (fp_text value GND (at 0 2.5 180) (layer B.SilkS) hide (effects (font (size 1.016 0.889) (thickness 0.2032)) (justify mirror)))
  (pad 1 thru_hole rect (at -4 0 180) (size 1.524 1.524) (drill 1) (layers *.Cu *.Mask B.SilkS) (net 1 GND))
  (pad 2 thru_hole circle (at -2 0 180) (size 1.524 1.524) (drill 1) (layers *.Cu *.Mask B.SilkS) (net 1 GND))
  (pad 3 thru_hole circle (at 0 0 180) (size 1.524 1.524) (drill 1) (layers *.Cu *.Mask B.SilkS) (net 1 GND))
  (pad 4 thru_hole circle (at 2 0 180) (size 1.524 1.524) (drill 1) (layers *.Cu *.Mask B.SilkS) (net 1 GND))
  (pad 5 thru_hole circle (at 4 0 180) (size 1.524 1.524) (drill 1) (layers *.Cu *.Mask B.SilkS) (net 1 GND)))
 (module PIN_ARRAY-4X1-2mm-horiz (layer F.Cu) (at 61.5 37)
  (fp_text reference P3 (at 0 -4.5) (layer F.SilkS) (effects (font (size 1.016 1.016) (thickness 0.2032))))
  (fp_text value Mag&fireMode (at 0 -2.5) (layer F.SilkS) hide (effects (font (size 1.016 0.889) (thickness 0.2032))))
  (pad 1 thru_hole rect (at -3 0) (size 1.524 1.524) (drill 1) (layers *.Cu *.Mask F.SilkS) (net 51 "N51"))
  (pad 2 thru_hole circle (at -1 0) (size 1.524 1.524) (drill 1) (layers *.Cu *.Mask F.SilkS) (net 52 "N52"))
  (pad 3 thru_hole circle (at 1 0) (size 1.524 1.524) (drill 1) (layers *.Cu *.Mask F.SilkS) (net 53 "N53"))
  (pad 4 thru_hole circle (at 3 0) (size 1.524 1.524) (drill 1) (layers *.Cu *.Mask F.SilkS) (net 54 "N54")))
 (gr_line (start 111.6 71.9) (end 62.5 71.9) (angle 90) (layer Edge.Cuts) (width 0.15))
 (segment (start 91.425 61.275) (end 91.425 60.875) (width 0.254) (layer F.Cu) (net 19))
 (segment (start 91.425 60.875) (end 92.1 60.2) (width 0.254) (layer F.Cu) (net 19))
 (segment (start 92.1 60.2) (end 92.7 60.2) (width 0.254) (layer F.Cu) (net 19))
 (segment (start 92.7 60.2) (end 92.9 60) (width 0.254) (layer F.Cu) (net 19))
 (segment (start 92.9 60) (end 92.9 59) (width 0.254) (layer F.Cu) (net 19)) (via (at 92.9 59) (size 0.6) (layers F.Cu B.Cu) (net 19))
 (segment (start 92.9 59) (end 93.8525 59) (width 0.254) (layer B.Cu) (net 19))
 (segment (start 88.5475 57.1) (end 88.5475 59) (width 0.254) (layer B.Cu) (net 24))
 (segment (start 91.425 54.925) (end 91.425 55.225) (width 0.254) (layer F.Cu) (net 21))
 (segment (start 92.7 55.9) (end 92.9 56.1) (width 0.254) (layer F.Cu) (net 21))
 (segment (start 92.9 56.1) (end 92.9 57.1) (width 0.254) (layer F.Cu) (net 21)) (via (at 92.9 57.1) (size 0.6) (layers F.Cu B.Cu) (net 21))
 (segment (start 92.9 57.1) (end 93.8525 57.1) (width 0.254) (layer B.Cu) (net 21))
 (segment (start 91.425 55.225) (end 92.1 55.9) (width 0.254) (layer F.Cu) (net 21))
 (segment (start 92.1 55.9) (end 92.7 55.9) (width 0.254) (layer F.Cu) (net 21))
 (segment (start 91.9475 57.1) (end 90.4525 57.1) (width 0.254) (layer B.Cu) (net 28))
 (segment (start 70.6 70.5) (end 69 70.5) (width 0.254) (layer F.Cu) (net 55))
 (segment (start 65.44 64.2) (end 66.77 62.87) (width 0.254) (layer F.Cu) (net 55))
 (segment (start 63.6 64.2) (end 65.44 64.2) (width 0.254) (layer F.Cu) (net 55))
 (segment (start 63 64.8) (end 63.6 64.2) (width 0.254) (layer F.Cu) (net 55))
 (segment (start 63 68.7) (end 63 64.8) (width 0.254) (layer F.Cu) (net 55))
 (segment (start 63.5 69.2) (end 63 68.7) (width 0.254) (layer F.Cu) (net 55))
 (segment (start 67.7 69.2) (end 63.5 69.2) (width 0.254) (layer F.Cu) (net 55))
 (segment (start 69 70.5) (end 67.7 69.2) (width 0.254) (layer F.Cu) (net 55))
 (segment (start 90.4525 59) (end 91.9475 59) (width 0.254) (layer B.Cu) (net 27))
 (segment (start 64.23 70.49) (end 64.23 70.53) (width 0.254) (layer F.Cu) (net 57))
 (segment (start 73.5 71.6) (end 74.6 70.5) (width 0.254) (layer F.Cu) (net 57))
 (segment (start 65.3 71.6) (end 73.5 71.6) (width 0.254) (layer F.Cu) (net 57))
 (segment (start 64.23 70.53) (end 65.3 71.6) (width 0.254) (layer F.Cu) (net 57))
 (segment (start 66.77 67.95) (end 71.15 67.95) (width 0.254) (layer F.Cu) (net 56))
 (segment (start 72.6 69.4) (end 72.6 70.5) (width 0.254) (layer F.Cu) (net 56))
 (segment (start 71.15 67.95) (end 72.6 69.4) (width 0.254) (layer F.Cu) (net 56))
 (segment (start 66.77 70.49) (end 67.783 70.49) (width 0.254) (layer B.Cu) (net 14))
 (segment (start 67.783 70.49) (end 69.584 68.689) (width 0.254) (layer B.Cu) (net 14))
 (segment (start 64.23 67.95) (end 64.25 67.95) (width 0.254) (layer B.Cu) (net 2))
 (segment (start 72.495 64.4) (end 73.411 63.484) (width 0.254) (layer B.Cu) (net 2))
 (segment (start 69.1 64.4) (end 72.495 64.4) (width 0.254) (layer B.Cu) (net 2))
 (segment (start 68.5 65) (end 69.1 64.4) (width 0.254) (layer B.Cu) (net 2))
 (segment (start 68.5 65.6) (end 68.5 65) (width 0.254) (layer B.Cu) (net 2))
 (segment (start 67.4 66.7) (end 68.5 65.6) (width 0.254) (layer B.Cu) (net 2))
 (segment (start 65.5 66.7) (end 67.4 66.7) (width 0.254) (layer B.Cu) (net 2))
 (segment (start 64.25 67.95) (end 65.5 66.7) (width 0.254) (layer B.Cu) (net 2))
 (segment (start 66.77 65.41) (end 66.814002 65.41) (width 0.254) (layer F.Cu) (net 4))
 (segment (start 74.389 68.789) (end 73.384 68.789) (width 0.254) (layer B.Cu) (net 4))
 (segment (start 74.6 69) (end 74.389 68.789) (width 0.254) (layer B.Cu) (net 4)) (via (at 74.6 69) (size 0.6) (layers F.Cu B.Cu) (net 4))
 (segment (start 73.095998 67.495998) (end 74.6 69) (width 0.254) (layer F.Cu) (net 4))
 (segment (start 68.9 67.495998) (end 73.095998 67.495998) (width 0.254) (layer F.Cu) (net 4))
 (segment (start 66.814002 65.41) (end 68.9 67.495998) (width 0.254) (layer F.Cu) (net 4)))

